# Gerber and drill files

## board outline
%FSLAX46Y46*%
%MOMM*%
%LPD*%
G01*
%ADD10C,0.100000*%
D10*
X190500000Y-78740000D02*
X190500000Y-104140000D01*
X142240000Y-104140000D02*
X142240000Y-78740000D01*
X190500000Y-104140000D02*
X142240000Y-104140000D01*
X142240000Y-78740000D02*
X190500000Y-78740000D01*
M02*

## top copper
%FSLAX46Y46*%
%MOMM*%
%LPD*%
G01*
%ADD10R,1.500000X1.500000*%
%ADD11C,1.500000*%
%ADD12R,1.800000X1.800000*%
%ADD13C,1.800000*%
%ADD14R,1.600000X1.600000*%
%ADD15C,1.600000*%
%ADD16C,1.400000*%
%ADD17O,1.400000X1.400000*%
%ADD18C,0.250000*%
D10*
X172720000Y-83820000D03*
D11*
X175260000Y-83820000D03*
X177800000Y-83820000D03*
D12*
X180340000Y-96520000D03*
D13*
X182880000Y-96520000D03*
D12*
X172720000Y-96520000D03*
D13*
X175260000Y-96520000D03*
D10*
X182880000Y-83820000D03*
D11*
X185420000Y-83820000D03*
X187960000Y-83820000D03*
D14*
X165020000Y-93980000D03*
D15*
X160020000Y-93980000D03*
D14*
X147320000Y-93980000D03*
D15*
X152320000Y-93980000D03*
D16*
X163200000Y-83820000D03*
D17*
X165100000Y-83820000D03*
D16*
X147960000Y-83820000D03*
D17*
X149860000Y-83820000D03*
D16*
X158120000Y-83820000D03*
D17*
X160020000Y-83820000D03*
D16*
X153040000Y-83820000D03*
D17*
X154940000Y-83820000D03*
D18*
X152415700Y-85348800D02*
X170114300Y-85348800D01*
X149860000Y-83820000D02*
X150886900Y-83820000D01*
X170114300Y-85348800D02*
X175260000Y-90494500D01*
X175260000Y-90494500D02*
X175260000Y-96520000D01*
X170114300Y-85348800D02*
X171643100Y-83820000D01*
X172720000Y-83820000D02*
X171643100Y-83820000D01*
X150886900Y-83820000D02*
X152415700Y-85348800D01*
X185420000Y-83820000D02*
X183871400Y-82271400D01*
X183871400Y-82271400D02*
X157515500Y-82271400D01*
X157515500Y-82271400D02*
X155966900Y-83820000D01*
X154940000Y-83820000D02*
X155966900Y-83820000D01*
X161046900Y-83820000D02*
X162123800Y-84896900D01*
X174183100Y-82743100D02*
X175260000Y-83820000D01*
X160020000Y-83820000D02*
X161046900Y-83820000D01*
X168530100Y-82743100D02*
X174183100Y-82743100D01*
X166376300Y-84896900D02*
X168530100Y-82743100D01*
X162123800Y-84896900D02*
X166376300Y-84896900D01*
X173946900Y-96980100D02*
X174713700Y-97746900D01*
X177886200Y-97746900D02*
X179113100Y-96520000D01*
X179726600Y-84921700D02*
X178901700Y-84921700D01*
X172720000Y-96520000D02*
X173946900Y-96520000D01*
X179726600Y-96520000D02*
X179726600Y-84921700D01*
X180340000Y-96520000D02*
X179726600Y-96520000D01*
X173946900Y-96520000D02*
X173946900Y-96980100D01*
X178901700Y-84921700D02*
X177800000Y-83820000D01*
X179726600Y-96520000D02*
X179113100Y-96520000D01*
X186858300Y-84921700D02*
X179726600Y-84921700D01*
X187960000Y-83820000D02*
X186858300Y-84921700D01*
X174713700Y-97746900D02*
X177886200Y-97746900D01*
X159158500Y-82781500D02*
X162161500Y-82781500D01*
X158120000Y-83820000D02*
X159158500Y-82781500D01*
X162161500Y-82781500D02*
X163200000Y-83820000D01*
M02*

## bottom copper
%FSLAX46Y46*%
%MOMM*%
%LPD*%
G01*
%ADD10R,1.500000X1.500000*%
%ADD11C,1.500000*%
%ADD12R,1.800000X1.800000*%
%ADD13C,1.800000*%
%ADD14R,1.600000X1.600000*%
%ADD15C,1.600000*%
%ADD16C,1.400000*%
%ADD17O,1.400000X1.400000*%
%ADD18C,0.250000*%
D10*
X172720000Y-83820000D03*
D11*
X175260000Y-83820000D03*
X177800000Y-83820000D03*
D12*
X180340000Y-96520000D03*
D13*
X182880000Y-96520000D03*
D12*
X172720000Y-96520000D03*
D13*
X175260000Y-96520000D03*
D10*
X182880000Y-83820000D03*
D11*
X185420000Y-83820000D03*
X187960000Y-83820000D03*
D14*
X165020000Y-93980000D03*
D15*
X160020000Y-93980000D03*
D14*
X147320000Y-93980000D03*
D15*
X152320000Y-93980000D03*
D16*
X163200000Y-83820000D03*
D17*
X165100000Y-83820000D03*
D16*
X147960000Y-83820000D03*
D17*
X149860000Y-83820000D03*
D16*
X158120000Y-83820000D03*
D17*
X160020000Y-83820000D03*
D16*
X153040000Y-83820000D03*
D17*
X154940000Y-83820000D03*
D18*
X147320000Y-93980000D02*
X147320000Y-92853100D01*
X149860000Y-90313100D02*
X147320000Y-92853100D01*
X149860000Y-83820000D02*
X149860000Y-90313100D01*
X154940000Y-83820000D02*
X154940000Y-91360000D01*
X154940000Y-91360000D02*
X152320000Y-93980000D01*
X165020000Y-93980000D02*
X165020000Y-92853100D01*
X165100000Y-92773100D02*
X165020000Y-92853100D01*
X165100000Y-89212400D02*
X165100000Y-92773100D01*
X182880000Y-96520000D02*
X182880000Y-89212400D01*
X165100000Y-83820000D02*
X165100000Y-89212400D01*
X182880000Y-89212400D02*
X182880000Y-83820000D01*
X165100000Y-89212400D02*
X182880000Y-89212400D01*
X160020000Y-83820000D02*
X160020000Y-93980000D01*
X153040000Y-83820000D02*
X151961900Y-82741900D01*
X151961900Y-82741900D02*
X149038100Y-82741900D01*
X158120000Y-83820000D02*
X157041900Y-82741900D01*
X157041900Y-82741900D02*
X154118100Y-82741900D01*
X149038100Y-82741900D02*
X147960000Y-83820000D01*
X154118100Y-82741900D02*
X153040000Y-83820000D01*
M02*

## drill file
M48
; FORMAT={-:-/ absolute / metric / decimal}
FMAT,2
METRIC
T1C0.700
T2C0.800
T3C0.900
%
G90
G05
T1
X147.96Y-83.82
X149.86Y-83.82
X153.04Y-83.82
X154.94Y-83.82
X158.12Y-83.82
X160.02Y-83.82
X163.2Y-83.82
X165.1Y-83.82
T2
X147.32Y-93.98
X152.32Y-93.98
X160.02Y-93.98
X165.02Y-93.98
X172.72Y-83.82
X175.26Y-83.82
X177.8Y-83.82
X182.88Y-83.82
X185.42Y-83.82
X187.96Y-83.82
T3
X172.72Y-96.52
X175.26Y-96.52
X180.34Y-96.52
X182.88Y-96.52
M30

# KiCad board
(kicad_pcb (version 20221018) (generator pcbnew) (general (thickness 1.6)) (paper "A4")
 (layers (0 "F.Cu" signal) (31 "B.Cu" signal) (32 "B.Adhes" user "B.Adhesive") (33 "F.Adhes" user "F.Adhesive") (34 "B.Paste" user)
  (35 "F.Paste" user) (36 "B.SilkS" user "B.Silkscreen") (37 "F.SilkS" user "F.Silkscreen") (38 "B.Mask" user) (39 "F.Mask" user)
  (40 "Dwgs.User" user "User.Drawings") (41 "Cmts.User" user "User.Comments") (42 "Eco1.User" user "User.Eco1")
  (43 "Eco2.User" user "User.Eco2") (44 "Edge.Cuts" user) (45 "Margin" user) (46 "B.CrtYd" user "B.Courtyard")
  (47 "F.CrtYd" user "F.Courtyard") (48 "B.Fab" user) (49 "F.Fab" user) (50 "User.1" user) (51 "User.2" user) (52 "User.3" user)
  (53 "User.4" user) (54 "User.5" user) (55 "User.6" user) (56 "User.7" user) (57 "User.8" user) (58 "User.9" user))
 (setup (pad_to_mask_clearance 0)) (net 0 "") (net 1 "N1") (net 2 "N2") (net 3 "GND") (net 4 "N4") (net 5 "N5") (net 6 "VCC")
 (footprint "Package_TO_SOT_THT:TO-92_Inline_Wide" (layer "F.Cu") (at 172.72 83.82)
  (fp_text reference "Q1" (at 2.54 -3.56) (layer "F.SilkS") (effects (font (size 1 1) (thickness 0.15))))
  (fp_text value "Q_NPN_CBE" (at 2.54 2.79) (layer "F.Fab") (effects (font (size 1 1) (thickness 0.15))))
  (pad "1" thru_hole rect (at 0 0) (size 1.5 1.5) (drill 0.8) (layers "*.Cu" "*.Mask") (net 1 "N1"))
  (pad "2" thru_hole circle (at 2.54 0) (size 1.5 1.5) (drill 0.8) (layers "*.Cu" "*.Mask") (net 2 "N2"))
  (pad "3" thru_hole circle (at 5.08 0) (size 1.5 1.5) (drill 0.8) (layers "*.Cu" "*.Mask") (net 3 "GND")))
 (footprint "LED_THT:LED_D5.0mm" (layer "F.Cu") (at 180.34 96.52)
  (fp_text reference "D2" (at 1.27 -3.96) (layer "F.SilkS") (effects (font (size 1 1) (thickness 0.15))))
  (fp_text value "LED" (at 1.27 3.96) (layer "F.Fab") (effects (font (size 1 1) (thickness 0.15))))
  (pad "1" thru_hole rect (at 0 0) (size 1.8 1.8) (drill 0.9) (layers "*.Cu" "*.Mask") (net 3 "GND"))
  (pad "2" thru_hole circle (at 2.54 0) (size 1.8 1.8) (drill 0.9) (layers "*.Cu" "*.Mask") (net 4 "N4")))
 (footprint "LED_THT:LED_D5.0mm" (layer "F.Cu") (at 172.72 96.52)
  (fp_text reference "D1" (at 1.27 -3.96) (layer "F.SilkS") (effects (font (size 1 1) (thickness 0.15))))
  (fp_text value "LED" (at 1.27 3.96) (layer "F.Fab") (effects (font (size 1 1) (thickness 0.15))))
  (pad "1" thru_hole rect (at 0 0) (size 1.8 1.8) (drill 0.9) (layers "*.Cu" "*.Mask") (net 3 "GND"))
  (pad "2" thru_hole circle (at 2.54 0) (size 1.8 1.8) (drill 0.9) (layers "*.Cu" "*.Mask") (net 1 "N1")))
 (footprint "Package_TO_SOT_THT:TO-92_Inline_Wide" (layer "F.Cu") (at 182.88 83.82)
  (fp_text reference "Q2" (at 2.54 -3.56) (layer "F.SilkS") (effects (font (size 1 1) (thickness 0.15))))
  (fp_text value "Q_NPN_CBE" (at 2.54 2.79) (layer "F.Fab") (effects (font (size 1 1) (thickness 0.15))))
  (pad "1" thru_hole rect (at 0 0) (size 1.5 1.5) (drill 0.8) (layers "*.Cu" "*.Mask") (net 4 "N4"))
  (pad "2" thru_hole circle (at 2.54 0) (size 1.5 1.5) (drill 0.8) (layers "*.Cu" "*.Mask") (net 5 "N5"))
  (pad "3" thru_hole circle (at 5.08 0) (size 1.5 1.5) (drill 0.8) (layers "*.Cu" "*.Mask") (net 3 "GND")))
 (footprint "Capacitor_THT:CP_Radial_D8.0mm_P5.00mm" (layer "F.Cu") (at 165.02 93.98 180)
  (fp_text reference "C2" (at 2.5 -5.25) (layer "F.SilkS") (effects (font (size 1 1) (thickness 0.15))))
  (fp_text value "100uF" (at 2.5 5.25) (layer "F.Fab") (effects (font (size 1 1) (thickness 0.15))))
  (pad "1" thru_hole rect (at 0 0 180) (size 1.6 1.6) (drill 0.8) (layers "*.Cu" "*.Mask") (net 4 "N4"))
  (pad "2" thru_hole circle (at 5 0 180) (size 1.6 1.6) (drill 0.8) (layers "*.Cu" "*.Mask") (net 2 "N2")))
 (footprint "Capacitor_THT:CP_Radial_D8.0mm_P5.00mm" (layer "F.Cu") (at 147.32 93.98)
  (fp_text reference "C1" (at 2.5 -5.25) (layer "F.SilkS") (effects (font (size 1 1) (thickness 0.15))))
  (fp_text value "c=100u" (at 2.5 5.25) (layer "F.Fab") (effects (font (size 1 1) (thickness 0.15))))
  (pad "1" thru_hole rect (at 0 0) (size 1.6 1.6) (drill 0.8) (layers "*.Cu" "*.Mask") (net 1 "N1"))
  (pad "2" thru_hole circle (at 5 0) (size 1.6 1.6) (drill 0.8) (layers "*.Cu" "*.Mask") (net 5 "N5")))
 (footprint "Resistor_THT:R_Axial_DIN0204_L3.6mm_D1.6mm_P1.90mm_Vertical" (layer "F.Cu") (at 163.2 83.82)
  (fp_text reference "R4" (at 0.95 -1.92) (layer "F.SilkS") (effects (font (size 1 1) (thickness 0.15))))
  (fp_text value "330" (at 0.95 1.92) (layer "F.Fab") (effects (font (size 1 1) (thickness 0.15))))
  (pad "1" thru_hole circle (at 0 0) (size 1.4 1.4) (drill 0.7) (layers "*.Cu" "*.Mask") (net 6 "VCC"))
  (pad "2" thru_hole oval (at 1.9 0) (size 1.4 1.4) (drill 0.7) (layers "*.Cu" "*.Mask") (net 4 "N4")))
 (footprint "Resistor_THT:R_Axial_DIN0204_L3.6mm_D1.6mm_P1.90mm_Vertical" (layer "F.Cu") (at 147.96 83.82)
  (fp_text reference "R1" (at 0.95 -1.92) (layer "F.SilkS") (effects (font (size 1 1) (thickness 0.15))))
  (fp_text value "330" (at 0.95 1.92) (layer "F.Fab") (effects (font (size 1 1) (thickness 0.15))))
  (pad "1" thru_hole circle (at 0 0) (size 1.4 1.4) (drill 0.7) (layers "*.Cu" "*.Mask") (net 6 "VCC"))
  (pad "2" thru_hole oval (at 1.9 0) (size 1.4 1.4) (drill 0.7) (layers "*.Cu" "*.Mask") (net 1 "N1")))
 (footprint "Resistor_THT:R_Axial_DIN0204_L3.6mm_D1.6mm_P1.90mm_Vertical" (layer "F.Cu") (at 158.12 83.82)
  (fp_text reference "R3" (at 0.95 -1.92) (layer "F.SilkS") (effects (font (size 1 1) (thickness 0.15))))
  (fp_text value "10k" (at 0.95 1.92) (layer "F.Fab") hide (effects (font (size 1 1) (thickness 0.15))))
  (pad "1" thru_hole circle (at 0 0) (size 1.4 1.4) (drill 0.7) (layers "*.Cu" "*.Mask") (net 6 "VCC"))
  (pad "2" thru_hole oval (at 1.9 0) (size 1.4 1.4) (drill 0.7) (layers "*.Cu" "*.Mask") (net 2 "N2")))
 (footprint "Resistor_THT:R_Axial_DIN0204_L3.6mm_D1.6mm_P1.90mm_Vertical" (layer "F.Cu") (at 153.04 83.82)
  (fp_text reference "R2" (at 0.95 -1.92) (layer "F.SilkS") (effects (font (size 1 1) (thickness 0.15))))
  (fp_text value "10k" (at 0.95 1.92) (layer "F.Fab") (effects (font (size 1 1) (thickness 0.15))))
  (pad "1" thru_hole circle (at 0 0) (size 1.4 1.4) (drill 0.7) (layers "*.Cu" "*.Mask") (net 6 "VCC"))
  (pad "2" thru_hole oval (at 1.9 0) (size 1.4 1.4) (drill 0.7) (layers "*.Cu" "*.Mask") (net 5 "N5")))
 (gr_line (start 190.5 78.74) (end 190.5 104.14) (stroke (width 0.1) (type default)) (layer "Edge.Cuts"))
 (gr_line (start 142.24 104.14) (end 142.24 78.74) (stroke (width 0.1) (type default)) (layer "Edge.Cuts"))
 (gr_line (start 190.5 104.14) (end 142.24 104.14) (stroke (width 0.1) (type default)) (layer "Edge.Cuts"))
 (gr_line (start 142.24 78.74) (end 190.5 78.74) (stroke (width 0.1) (type default)) (layer "Edge.Cuts"))
 (segment (start 152.4157 85.3488) (end 170.1143 85.3488) (width 0.25) (layer "F.Cu") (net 1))
 (segment (start 149.86 83.82) (end 150.8869 83.82) (width 0.25) (layer "F.Cu") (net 1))
 (segment (start 170.1143 85.3488) (end 175.26 90.4945) (width 0.25) (layer "F.Cu") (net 1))
 (segment (start 175.26 90.4945) (end 175.26 96.52) (width 0.25) (layer "F.Cu") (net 1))
 (segment (start 170.1143 85.3488) (end 171.6431 83.82) (width 0.25) (layer "F.Cu") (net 1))
 (segment (start 172.72 83.82) (end 171.6431 83.82) (width 0.25) (layer "F.Cu") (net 1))
 (segment (start 150.8869 83.82) (end 152.4157 85.3488) (width 0.25) (layer "F.Cu") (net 1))
 (segment (start 147.32 93.98) (end 147.32 92.8531) (width 0.25) (layer "B.Cu") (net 1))
 (segment (start 149.86 90.3131) (end 147.32 92.8531) (width 0.25) (layer "B.Cu") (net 1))
 (segment (start 149.86 83.82) (end 149.86 90.3131) (width 0.25) (layer "B.Cu") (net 1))
 (segment (start 185.42 83.82) (end 183.8714 82.2714) (width 0.25) (layer "F.Cu") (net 5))
 (segment (start 183.8714 82.2714) (end 157.5155 82.2714) (width 0.25) (layer "F.Cu") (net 5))
 (segment (start 157.5155 82.2714) (end 155.9669 83.82) (width 0.25) (layer "F.Cu") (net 5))
 (segment (start 154.94 83.82) (end 155.9669 83.82) (width 0.25) (layer "F.Cu") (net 5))
 (segment (start 154.94 83.82) (end 154.94 91.36) (width 0.25) (layer "B.Cu") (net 5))
 (segment (start 154.94 91.36) (end 152.32 93.98) (width 0.25) (layer "B.Cu") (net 5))
 (segment (start 165.02 93.98) (end 165.02 92.8531) (width 0.25) (layer "B.Cu") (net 4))
 (segment (start 165.1 92.7731) (end 165.02 92.8531) (width 0.25) (layer "B.Cu") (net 4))
 (segment (start 165.1 89.2124) (end 165.1 92.7731) (width 0.25) (layer "B.Cu") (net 4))
 (segment (start 182.88 96.52) (end 182.88 89.2124) (width 0.25) (layer "B.Cu") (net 4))
 (segment (start 165.1 83.82) (end 165.1 89.2124) (width 0.25) (layer "B.Cu") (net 4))
 (segment (start 182.88 89.2124) (end 182.88 83.82) (width 0.25) (layer "B.Cu") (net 4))
 (segment (start 165.1 89.2124) (end 182.88 89.2124) (width 0.25) (layer "B.Cu") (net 4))
 (segment (start 161.0469 83.82) (end 162.1238 84.8969) (width 0.25) (layer "F.Cu") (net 2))
 (segment (start 174.1831 82.7431) (end 175.26 83.82) (width 0.25) (layer "F.Cu") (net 2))
 (segment (start 160.02 83.82) (end 161.0469 83.82) (width 0.25) (layer "F.Cu") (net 2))
 (segment (start 168.5301 82.7431) (end 174.1831 82.7431) (width 0.25) (layer "F.Cu") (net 2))
 (segment (start 166.3763 84.8969) (end 168.5301 82.7431) (width 0.25) (layer "F.Cu") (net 2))
 (segment (start 162.1238 84.8969) (end 166.3763 84.8969) (width 0.25) (layer "F.Cu") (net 2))
 (segment (start 160.02 83.82) (end 160.02 93.98) (width 0.25) (layer "B.Cu") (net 2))
 (segment (start 173.9469 96.9801) (end 174.7137 97.7469) (width 0.25) (layer "F.Cu") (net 3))
 (segment (start 177.8862 97.7469) (end 179.1131 96.52) (width 0.25) (layer "F.Cu") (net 3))
 (segment (start 179.7266 84.9217) (end 178.9017 84.9217) (width 0.25) (layer "F.Cu") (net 3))
 (segment (start 172.72 96.52) (end 173.9469 96.52) (width 0.25) (layer "F.Cu") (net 3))
 (segment (start 179.7266 96.52) (end 179.7266 84.9217) (width 0.25) (layer "F.Cu") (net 3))
 (segment (start 180.34 96.52) (end 179.7266 96.52) (width 0.25) (layer "F.Cu") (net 3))
 (segment (start 173.9469 96.52) (end 173.9469 96.9801) (width 0.25) (layer "F.Cu") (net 3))
 (segment (start 178.9017 84.9217) (end 177.8 83.82) (width 0.25) (layer "F.Cu") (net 3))
 (segment (start 179.7266 96.52) (end 179.1131 96.52) (width 0.25) (layer "F.Cu") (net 3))
 (segment (start 186.8583 84.9217) (end 179.7266 84.9217) (width 0.25) (layer "F.Cu") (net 3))
 (segment (start 187.96 83.82) (end 186.8583 84.9217) (width 0.25) (layer "F.Cu") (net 3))
 (segment (start 174.7137 97.7469) (end 177.8862 97.7469) (width 0.25) (layer "F.Cu") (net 3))
 (segment (start 159.1585 82.7815) (end 162.1615 82.7815) (width 0.25) (layer "F.Cu") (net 6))
 (segment (start 158.12 83.82) (end 159.1585 82.7815) (width 0.25) (layer "F.Cu") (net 6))
 (segment (start 162.1615 82.7815) (end 163.2 83.82) (width 0.25) (layer "F.Cu") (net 6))
 (segment (start 153.04 83.82) (end 151.9619 82.7419) (width 0.25) (layer "B.Cu") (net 6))
 (segment (start 151.9619 82.7419) (end 149.0381 82.7419) (width 0.25) (layer "B.Cu") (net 6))
 (segment (start 158.12 83.82) (end 157.0419 82.7419) (width 0.25) (layer "B.Cu") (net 6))
 (segment (start 157.0419 82.7419) (end 154.1181 82.7419) (width 0.25) (layer "B.Cu") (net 6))
 (segment (start 149.0381 82.7419) (end 147.96 83.82) (width 0.25) (layer "B.Cu") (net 6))
 (segment (start 154.1181 82.7419) (end 153.04 83.82) (width 0.25) (layer "B.Cu") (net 6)))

